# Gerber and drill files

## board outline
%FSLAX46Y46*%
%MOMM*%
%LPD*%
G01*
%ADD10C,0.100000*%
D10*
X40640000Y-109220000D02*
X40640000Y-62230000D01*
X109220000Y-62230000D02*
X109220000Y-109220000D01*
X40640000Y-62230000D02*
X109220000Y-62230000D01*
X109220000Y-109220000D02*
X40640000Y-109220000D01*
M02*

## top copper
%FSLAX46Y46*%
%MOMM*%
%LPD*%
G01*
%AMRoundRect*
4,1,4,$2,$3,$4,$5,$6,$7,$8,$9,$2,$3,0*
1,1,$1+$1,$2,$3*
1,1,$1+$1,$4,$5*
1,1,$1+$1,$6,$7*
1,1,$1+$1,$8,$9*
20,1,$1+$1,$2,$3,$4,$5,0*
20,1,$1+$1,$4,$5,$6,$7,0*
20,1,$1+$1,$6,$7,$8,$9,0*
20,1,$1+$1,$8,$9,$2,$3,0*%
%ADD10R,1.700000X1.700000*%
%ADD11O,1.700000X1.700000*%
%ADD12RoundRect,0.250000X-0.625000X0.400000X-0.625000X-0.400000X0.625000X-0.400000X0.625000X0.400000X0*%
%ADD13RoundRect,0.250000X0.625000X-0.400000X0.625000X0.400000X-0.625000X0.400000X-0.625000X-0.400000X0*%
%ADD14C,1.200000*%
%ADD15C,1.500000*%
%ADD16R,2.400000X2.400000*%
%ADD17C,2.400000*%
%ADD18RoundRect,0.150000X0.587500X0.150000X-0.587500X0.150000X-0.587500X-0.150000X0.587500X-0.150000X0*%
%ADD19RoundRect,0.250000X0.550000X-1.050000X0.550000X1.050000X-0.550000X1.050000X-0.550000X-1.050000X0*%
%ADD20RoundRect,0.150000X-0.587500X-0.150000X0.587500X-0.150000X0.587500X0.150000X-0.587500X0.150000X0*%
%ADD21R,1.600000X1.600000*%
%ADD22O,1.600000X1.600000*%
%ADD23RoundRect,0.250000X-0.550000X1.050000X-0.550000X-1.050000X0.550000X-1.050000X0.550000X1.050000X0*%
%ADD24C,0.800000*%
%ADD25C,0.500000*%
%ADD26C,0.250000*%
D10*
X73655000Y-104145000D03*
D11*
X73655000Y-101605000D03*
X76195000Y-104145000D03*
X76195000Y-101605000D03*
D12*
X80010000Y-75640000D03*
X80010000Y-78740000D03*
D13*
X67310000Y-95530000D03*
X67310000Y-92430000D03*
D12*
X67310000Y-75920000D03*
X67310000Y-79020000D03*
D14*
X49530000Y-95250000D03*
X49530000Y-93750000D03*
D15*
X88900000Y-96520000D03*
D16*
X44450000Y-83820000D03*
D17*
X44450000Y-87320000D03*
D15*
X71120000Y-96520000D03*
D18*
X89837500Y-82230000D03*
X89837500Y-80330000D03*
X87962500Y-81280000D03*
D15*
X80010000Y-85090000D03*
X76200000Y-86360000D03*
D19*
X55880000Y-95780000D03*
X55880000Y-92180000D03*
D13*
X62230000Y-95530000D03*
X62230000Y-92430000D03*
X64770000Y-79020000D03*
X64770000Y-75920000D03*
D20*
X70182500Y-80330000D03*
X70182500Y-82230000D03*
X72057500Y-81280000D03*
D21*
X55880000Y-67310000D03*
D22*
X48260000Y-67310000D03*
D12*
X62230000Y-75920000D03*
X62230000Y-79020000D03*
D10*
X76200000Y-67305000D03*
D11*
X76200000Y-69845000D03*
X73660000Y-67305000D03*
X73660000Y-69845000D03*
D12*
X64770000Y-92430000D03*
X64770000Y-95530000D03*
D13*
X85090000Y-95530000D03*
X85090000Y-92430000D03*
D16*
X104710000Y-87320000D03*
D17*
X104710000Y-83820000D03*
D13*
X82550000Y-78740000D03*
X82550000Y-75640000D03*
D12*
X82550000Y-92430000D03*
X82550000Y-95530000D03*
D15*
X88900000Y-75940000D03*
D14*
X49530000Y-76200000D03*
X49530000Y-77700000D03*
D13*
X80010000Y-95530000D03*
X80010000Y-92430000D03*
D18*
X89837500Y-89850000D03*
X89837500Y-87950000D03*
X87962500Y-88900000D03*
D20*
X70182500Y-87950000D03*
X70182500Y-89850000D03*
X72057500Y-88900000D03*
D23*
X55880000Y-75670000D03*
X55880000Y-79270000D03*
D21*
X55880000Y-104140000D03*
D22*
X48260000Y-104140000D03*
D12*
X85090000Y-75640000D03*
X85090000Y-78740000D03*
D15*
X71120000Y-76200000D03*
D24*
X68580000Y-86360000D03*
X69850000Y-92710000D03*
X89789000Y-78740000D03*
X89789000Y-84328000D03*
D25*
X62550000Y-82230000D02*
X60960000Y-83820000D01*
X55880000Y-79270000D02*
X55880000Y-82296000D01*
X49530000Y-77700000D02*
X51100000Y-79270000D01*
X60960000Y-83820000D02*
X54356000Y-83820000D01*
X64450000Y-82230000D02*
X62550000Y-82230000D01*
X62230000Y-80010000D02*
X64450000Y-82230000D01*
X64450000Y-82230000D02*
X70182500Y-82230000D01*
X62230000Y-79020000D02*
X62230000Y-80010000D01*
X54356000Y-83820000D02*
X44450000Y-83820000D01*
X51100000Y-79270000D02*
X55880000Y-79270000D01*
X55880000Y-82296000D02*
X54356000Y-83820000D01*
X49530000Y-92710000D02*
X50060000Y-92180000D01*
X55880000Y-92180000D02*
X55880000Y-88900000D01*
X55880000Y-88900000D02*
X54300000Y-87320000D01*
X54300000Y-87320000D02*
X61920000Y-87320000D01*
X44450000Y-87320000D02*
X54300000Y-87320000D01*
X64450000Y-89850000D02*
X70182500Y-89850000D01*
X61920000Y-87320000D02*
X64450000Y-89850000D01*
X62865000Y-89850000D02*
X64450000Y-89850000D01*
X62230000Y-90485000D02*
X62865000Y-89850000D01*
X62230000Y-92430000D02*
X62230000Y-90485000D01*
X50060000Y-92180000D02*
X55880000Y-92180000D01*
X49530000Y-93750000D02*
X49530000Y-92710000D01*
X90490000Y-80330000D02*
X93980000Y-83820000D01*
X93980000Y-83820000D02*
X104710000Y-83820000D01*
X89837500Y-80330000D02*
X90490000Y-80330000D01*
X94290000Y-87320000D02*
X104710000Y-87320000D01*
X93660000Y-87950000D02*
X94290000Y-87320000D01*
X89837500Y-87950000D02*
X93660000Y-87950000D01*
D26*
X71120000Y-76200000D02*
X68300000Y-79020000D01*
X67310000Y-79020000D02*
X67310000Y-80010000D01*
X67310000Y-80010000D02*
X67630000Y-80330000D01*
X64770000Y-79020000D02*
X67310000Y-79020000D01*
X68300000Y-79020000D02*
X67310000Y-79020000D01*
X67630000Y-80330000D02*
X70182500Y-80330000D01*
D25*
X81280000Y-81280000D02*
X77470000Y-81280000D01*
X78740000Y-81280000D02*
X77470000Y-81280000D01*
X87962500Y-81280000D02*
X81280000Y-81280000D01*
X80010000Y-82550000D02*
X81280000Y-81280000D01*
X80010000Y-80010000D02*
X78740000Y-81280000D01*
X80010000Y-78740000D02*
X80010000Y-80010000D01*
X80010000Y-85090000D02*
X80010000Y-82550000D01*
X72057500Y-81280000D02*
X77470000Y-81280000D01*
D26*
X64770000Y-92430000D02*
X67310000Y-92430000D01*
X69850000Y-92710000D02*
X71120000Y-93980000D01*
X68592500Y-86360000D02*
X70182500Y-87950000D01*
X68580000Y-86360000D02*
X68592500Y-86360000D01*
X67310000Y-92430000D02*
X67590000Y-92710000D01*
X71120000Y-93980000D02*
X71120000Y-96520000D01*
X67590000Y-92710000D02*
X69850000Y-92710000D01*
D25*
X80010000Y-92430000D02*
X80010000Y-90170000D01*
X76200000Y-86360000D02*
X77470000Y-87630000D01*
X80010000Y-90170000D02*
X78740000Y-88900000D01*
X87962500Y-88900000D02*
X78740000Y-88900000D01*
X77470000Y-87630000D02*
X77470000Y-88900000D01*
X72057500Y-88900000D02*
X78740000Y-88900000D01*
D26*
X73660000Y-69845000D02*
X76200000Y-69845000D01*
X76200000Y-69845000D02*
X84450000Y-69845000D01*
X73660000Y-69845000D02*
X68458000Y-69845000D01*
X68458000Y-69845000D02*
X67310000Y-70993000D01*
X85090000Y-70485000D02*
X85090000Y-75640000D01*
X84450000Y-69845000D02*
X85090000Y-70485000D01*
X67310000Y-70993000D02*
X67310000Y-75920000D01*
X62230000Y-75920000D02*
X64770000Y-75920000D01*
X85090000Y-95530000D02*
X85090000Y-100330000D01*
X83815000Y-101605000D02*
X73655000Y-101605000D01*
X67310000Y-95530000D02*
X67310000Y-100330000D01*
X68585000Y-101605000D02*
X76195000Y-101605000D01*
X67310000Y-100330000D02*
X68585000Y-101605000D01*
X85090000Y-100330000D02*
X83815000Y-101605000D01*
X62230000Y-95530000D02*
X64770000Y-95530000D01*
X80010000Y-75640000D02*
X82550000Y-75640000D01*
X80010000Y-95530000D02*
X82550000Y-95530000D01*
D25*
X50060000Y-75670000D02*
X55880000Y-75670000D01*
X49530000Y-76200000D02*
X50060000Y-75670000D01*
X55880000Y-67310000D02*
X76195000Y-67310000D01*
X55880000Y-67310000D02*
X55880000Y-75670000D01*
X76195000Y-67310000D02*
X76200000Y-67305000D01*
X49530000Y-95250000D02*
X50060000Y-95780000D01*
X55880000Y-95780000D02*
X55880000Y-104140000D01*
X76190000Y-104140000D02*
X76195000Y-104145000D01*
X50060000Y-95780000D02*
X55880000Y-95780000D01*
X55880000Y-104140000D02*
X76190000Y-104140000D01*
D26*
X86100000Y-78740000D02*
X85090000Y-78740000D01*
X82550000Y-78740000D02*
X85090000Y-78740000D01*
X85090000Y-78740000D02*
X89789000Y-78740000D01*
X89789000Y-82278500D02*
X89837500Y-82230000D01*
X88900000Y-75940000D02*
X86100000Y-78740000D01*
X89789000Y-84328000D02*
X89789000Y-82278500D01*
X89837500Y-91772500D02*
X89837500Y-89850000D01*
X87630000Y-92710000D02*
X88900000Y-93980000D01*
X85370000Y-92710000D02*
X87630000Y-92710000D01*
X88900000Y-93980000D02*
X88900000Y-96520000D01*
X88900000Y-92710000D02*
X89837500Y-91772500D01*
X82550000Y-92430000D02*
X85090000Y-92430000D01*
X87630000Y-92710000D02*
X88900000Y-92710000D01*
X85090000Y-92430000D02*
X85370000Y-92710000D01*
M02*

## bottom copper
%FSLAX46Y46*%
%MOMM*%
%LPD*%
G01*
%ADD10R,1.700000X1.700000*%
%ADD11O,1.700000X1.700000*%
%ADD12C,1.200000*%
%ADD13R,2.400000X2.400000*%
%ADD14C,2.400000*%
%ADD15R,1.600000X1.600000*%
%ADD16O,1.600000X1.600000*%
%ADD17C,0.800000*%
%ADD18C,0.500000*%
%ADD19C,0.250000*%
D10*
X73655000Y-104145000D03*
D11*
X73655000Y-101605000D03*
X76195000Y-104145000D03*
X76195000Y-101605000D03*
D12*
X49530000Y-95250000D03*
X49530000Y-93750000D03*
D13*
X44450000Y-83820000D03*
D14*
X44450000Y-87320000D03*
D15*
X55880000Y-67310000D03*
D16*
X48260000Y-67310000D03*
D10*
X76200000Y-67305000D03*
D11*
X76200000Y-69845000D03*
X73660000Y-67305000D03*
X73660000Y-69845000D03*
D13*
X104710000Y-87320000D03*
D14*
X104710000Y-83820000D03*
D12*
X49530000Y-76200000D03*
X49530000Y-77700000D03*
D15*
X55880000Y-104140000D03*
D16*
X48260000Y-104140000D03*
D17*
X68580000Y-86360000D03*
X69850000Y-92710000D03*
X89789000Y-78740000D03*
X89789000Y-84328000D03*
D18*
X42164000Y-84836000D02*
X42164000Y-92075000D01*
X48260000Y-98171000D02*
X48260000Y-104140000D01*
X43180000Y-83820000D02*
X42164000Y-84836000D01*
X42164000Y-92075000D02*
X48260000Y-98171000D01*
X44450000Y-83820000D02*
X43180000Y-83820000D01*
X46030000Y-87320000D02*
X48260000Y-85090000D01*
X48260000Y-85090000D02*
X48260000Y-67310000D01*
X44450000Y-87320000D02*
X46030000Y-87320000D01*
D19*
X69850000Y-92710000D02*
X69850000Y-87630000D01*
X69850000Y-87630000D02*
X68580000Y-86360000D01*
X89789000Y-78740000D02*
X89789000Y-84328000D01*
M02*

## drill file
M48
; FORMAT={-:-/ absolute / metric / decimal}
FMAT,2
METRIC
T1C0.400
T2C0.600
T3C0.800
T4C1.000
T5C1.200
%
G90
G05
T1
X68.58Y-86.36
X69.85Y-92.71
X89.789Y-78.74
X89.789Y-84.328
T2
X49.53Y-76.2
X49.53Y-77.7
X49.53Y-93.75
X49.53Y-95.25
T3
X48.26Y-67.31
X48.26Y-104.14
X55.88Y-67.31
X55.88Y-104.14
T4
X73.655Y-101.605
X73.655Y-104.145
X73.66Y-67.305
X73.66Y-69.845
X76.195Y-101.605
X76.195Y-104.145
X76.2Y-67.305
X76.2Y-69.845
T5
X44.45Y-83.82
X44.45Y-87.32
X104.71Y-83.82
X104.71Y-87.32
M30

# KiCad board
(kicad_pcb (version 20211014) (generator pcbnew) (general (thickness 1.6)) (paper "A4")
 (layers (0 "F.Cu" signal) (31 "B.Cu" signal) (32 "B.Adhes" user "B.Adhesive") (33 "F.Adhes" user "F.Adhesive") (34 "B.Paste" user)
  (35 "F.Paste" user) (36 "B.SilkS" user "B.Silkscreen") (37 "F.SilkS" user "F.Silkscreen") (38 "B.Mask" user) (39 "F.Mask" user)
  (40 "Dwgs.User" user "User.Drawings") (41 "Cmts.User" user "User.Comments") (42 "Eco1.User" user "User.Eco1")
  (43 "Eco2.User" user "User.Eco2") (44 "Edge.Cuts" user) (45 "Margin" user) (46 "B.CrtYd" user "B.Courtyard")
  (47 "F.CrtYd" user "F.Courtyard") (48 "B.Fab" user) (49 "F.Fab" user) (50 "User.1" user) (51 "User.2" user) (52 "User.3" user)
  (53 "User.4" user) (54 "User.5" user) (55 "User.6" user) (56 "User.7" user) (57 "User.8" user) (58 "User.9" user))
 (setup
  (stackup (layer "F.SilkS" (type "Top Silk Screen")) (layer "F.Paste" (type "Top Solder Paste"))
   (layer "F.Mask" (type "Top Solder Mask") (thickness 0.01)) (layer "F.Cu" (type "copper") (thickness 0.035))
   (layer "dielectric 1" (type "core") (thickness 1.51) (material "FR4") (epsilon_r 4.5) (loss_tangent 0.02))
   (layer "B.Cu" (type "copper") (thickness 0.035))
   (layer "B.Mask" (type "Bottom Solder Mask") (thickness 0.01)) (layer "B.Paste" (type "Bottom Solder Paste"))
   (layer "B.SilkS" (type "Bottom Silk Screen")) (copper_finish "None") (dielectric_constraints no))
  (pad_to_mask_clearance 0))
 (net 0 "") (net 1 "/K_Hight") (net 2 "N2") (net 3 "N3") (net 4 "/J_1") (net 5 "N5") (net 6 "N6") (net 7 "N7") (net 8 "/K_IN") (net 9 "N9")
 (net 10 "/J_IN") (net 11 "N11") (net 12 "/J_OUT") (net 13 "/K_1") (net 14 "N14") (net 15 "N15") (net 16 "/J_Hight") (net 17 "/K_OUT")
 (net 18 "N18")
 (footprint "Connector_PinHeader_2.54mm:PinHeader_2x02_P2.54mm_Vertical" (layer "F.Cu") (at 73.655 104.145 90)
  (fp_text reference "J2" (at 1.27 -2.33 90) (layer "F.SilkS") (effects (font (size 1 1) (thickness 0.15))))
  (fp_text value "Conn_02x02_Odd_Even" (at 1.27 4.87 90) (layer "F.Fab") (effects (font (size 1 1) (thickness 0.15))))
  (pad "1" thru_hole rect locked (at 0 0 90) (size 1.7 1.7) (drill 1) (layers *.Cu *.Mask) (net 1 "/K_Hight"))
  (pad "2" thru_hole oval locked (at 2.54 0 90) (size 1.7 1.7) (drill 1) (layers *.Cu *.Mask) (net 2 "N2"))
  (pad "3" thru_hole oval locked (at 0 2.54 90) (size 1.7 1.7) (drill 1) (layers *.Cu *.Mask) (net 1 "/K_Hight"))
  (pad "4" thru_hole oval locked (at 2.54 2.54 90) (size 1.7 1.7) (drill 1) (layers *.Cu *.Mask) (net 2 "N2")))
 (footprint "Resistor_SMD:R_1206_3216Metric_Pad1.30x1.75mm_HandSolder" (layer "F.Cu") (at 80.01 77.19 -90)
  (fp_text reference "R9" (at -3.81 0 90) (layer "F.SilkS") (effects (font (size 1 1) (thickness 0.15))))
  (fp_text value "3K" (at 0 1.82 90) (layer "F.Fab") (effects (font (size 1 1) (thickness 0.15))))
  (pad "1" smd roundrect locked (at -1.55 0 270) (size 1.3 1.75) (layers "F.Cu" "F.Paste" "F.Mask") (roundrect_rratio 0.1923076923)
   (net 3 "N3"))
  (pad "2" smd roundrect locked (at 1.55 0 270) (size 1.3 1.75) (layers "F.Cu" "F.Paste" "F.Mask") (roundrect_rratio 0.1923076923)
   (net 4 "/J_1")))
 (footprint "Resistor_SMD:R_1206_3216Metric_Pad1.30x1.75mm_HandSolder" (layer "F.Cu") (at 67.31 93.98 90)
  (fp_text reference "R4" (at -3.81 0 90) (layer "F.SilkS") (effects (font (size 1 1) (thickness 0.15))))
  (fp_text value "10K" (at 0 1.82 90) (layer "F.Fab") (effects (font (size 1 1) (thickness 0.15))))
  (pad "1" smd roundrect locked (at -1.55 0 90) (size 1.3 1.75) (layers "F.Cu" "F.Paste" "F.Mask") (roundrect_rratio 0.1923076923)
   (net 2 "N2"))
  (pad "2" smd roundrect locked (at 1.55 0 90) (size 1.3 1.75) (layers "F.Cu" "F.Paste" "F.Mask") (roundrect_rratio 0.1923076923)
   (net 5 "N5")))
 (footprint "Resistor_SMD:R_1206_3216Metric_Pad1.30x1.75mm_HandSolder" (layer "F.Cu") (at 67.31 77.47 -90)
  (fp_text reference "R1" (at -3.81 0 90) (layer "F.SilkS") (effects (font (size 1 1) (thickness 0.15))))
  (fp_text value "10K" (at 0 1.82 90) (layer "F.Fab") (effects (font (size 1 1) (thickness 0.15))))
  (pad "1" smd roundrect locked (at -1.55 0 270) (size 1.3 1.75) (layers "F.Cu" "F.Paste" "F.Mask") (roundrect_rratio 0.1923076923)
   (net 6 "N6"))
  (pad "2" smd roundrect locked (at 1.55 0 270) (size 1.3 1.75) (layers "F.Cu" "F.Paste" "F.Mask") (roundrect_rratio 0.1923076923)
   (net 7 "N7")))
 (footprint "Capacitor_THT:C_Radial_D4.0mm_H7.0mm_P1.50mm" (layer "F.Cu") (at 49.53 95.25 90)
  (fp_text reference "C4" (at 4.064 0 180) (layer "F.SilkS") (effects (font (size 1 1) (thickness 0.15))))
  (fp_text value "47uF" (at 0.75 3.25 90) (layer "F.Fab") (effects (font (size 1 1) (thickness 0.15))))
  (pad "1" thru_hole circle locked (at 0 0 90) (size 1.2 1.2) (drill 0.6) (layers *.Cu *.Mask) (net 1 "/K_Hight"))
  (pad "2" thru_hole circle locked (at 1.5 0 90) (size 1.2 1.2) (drill 0.6) (layers *.Cu *.Mask) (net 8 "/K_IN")))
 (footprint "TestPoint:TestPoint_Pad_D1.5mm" (layer "F.Cu") (at 88.9 96.52)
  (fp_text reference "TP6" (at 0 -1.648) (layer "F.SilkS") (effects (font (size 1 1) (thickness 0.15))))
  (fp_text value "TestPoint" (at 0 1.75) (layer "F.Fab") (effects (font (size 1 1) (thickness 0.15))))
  (pad "1" smd circle locked (at 0 0) (size 1.5 1.5) (layers "F.Cu" "F.Mask") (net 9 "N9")))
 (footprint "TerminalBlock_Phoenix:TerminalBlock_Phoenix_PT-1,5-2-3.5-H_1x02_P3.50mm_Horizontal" (layer "F.Cu") (at 44.45 83.82 -90)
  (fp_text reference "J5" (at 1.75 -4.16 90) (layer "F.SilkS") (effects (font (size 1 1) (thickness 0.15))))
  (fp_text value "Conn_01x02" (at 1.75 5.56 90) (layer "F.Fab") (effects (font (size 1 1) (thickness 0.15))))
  (pad "1" thru_hole rect locked (at 0 0 270) (size 2.4 2.4) (drill 1.2) (layers *.Cu *.Mask) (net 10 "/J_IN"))
  (pad "2" thru_hole circle locked (at 3.5 0 270) (size 2.4 2.4) (drill 1.2) (layers *.Cu *.Mask) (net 8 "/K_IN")))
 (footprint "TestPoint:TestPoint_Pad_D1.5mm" (layer "F.Cu") (at 71.12 96.52)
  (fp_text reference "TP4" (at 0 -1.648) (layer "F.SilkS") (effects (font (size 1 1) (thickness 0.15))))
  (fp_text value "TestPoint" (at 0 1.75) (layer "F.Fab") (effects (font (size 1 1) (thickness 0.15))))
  (pad "1" smd circle locked (at 0 0) (size 1.5 1.5) (layers "F.Cu" "F.Mask") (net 5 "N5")))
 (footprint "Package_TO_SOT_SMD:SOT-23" (layer "F.Cu") (at 88.9 81.28 180)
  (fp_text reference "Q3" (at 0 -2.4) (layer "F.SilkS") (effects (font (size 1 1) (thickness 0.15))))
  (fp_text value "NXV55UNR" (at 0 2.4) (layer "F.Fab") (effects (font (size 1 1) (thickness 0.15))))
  (pad "1" smd roundrect locked (at -0.9375 -0.95 180) (size 1.475 0.6) (layers "F.Cu" "F.Paste" "F.Mask") (roundrect_rratio 0.25)
   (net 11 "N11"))
  (pad "2" smd roundrect locked (at -0.9375 0.95 180) (size 1.475 0.6) (layers "F.Cu" "F.Paste" "F.Mask") (roundrect_rratio 0.25)
   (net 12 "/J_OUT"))
  (pad "3" smd roundrect locked (at 0.9375 0 180) (size 1.475 0.6) (layers "F.Cu" "F.Paste" "F.Mask") (roundrect_rratio 0.25) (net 4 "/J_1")))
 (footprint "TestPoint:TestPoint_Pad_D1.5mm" (layer "F.Cu") (at 80.01 85.09)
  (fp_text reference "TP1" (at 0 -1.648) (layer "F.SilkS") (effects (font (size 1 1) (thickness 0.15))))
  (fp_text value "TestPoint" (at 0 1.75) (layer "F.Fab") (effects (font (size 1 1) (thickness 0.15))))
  (pad "1" smd circle locked (at 0 0) (size 1.5 1.5) (layers "F.Cu" "F.Mask") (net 4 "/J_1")))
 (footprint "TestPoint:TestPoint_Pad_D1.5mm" (layer "F.Cu") (at 76.2 86.36)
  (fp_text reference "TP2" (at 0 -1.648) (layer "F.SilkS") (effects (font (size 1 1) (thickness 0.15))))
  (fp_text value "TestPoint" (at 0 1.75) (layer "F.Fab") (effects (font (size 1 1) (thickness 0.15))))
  (pad "1" smd circle locked (at 0 0) (size 1.5 1.5) (layers "F.Cu" "F.Mask") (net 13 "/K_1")))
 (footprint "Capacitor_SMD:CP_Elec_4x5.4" (layer "F.Cu") (at 55.88 93.98 90)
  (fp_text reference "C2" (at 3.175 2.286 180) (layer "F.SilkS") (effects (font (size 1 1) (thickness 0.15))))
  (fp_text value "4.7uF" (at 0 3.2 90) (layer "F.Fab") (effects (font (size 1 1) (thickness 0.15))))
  (pad "1" smd roundrect locked (at -1.8 0 90) (size 2.6 1.6) (layers "F.Cu" "F.Paste" "F.Mask") (roundrect_rratio 0.15625)
   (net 1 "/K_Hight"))
  (pad "2" smd roundrect locked (at 1.8 0 90) (size 2.6 1.6) (layers "F.Cu" "F.Paste" "F.Mask") (roundrect_rratio 0.15625) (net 8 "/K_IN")))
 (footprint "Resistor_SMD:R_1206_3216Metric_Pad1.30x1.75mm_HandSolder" (layer "F.Cu") (at 62.23 93.98 90)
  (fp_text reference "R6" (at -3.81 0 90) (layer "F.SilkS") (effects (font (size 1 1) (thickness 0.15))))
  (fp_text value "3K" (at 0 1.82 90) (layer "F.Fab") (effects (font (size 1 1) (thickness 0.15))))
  (pad "1" smd roundrect locked (at -1.55 0 90) (size 1.3 1.75) (layers "F.Cu" "F.Paste" "F.Mask") (roundrect_rratio 0.1923076923)
   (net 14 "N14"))
  (pad "2" smd roundrect locked (at 1.55 0 90) (size 1.3 1.75) (layers "F.Cu" "F.Paste" "F.Mask") (roundrect_rratio 0.1923076923)
   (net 8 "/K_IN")))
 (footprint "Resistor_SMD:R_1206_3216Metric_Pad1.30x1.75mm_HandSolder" (layer "F.Cu") (at 64.77 77.47 90)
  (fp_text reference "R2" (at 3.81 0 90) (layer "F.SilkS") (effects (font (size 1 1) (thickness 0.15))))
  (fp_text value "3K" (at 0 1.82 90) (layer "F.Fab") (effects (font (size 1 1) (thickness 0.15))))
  (pad "1" smd roundrect locked (at -1.55 0 90) (size 1.3 1.75) (layers "F.Cu" "F.Paste" "F.Mask") (roundrect_rratio 0.1923076923)
   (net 7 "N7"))
  (pad "2" smd roundrect locked (at 1.55 0 90) (size 1.3 1.75) (layers "F.Cu" "F.Paste" "F.Mask") (roundrect_rratio 0.1923076923)
   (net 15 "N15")))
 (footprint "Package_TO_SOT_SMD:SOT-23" (layer "F.Cu") (at 71.12 81.28)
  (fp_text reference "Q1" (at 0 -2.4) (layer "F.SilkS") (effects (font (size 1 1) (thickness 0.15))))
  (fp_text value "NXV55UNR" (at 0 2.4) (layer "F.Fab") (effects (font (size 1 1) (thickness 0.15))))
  (pad "1" smd roundrect locked (at -0.9375 -0.95) (size 1.475 0.6) (layers "F.Cu" "F.Paste" "F.Mask") (roundrect_rratio 0.25) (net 7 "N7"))
  (pad "2" smd roundrect locked (at -0.9375 0.95) (size 1.475 0.6) (layers "F.Cu" "F.Paste" "F.Mask") (roundrect_rratio 0.25)
   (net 10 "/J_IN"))
  (pad "3" smd roundrect locked (at 0.9375 0) (size 1.475 0.6) (layers "F.Cu" "F.Paste" "F.Mask") (roundrect_rratio 0.25) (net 4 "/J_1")))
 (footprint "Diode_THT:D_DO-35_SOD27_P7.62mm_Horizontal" (layer "F.Cu") (at 55.88 67.31 180)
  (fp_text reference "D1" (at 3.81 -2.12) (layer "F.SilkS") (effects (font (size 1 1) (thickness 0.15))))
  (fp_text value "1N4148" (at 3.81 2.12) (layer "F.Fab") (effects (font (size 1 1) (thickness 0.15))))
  (pad "1" thru_hole rect locked (at 0 0 180) (size 1.6 1.6) (drill 0.8) (layers *.Cu *.Mask) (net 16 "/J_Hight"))
  (pad "2" thru_hole oval locked (at 7.62 0 180) (size 1.6 1.6) (drill 0.8) (layers *.Cu *.Mask) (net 8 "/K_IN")))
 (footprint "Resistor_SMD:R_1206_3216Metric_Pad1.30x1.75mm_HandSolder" (layer "F.Cu") (at 62.23 77.47 -90)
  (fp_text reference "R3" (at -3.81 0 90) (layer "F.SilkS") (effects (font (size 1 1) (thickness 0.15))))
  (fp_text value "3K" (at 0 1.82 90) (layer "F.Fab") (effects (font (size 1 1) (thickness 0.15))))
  (pad "1" smd roundrect locked (at -1.55 0 270) (size 1.3 1.75) (layers "F.Cu" "F.Paste" "F.Mask") (roundrect_rratio 0.1923076923)
   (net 15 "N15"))
  (pad "2" smd roundrect locked (at 1.55 0 270) (size 1.3 1.75) (layers "F.Cu" "F.Paste" "F.Mask") (roundrect_rratio 0.1923076923)
   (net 10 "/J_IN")))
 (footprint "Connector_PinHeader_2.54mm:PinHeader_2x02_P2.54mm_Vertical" (layer "F.Cu") (at 76.2 67.305 -90) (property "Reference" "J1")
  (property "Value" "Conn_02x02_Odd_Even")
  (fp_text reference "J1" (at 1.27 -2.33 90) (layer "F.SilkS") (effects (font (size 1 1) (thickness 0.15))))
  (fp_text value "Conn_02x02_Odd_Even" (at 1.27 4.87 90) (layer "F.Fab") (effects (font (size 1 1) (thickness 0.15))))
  (pad "1" thru_hole rect locked (at 0 0 270) (size 1.7 1.7) (drill 1) (layers *.Cu *.Mask) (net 16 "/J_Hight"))
  (pad "2" thru_hole oval locked (at 2.54 0 270) (size 1.7 1.7) (drill 1) (layers *.Cu *.Mask) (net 6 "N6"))
  (pad "3" thru_hole oval locked (at 0 2.54 270) (size 1.7 1.7) (drill 1) (layers *.Cu *.Mask) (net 16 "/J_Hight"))
  (pad "4" thru_hole oval locked (at 2.54 2.54 270) (size 1.7 1.7) (drill 1) (layers *.Cu *.Mask) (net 6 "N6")))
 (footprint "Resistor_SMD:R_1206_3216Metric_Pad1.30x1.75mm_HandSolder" (layer "F.Cu") (at 64.77 93.98 -90)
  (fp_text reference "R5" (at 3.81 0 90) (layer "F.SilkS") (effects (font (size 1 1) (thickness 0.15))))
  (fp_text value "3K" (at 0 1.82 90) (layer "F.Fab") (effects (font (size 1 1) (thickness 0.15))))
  (pad "1" smd roundrect locked (at -1.55 0 270) (size 1.3 1.75) (layers "F.Cu" "F.Paste" "F.Mask") (roundrect_rratio 0.1923076923)
   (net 5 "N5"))
  (pad "2" smd roundrect locked (at 1.55 0 270) (size 1.3 1.75) (layers "F.Cu" "F.Paste" "F.Mask") (roundrect_rratio 0.1923076923)
   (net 14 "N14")))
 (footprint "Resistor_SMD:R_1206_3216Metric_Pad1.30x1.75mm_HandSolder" (layer "F.Cu") (at 85.09 93.98 90)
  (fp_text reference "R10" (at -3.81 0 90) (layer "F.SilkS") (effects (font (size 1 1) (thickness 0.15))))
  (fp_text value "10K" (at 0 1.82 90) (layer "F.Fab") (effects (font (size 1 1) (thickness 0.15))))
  (pad "1" smd roundrect locked (at -1.55 0 90) (size 1.3 1.75) (layers "F.Cu" "F.Paste" "F.Mask") (roundrect_rratio 0.1923076923)
   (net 2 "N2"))
  (pad "2" smd roundrect locked (at 1.55 0 90) (size 1.3 1.75) (layers "F.Cu" "F.Paste" "F.Mask") (roundrect_rratio 0.1923076923)
   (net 9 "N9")))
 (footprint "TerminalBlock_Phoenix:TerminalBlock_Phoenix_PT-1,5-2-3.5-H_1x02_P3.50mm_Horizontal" (layer "F.Cu") (at 104.71 87.32 90)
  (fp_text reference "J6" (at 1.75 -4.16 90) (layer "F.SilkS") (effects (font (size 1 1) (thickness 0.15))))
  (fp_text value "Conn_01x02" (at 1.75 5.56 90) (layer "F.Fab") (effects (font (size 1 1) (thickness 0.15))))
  (pad "1" thru_hole rect locked (at 0 0 90) (size 2.4 2.4) (drill 1.2) (layers *.Cu *.Mask) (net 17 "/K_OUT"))
  (pad "2" thru_hole circle locked (at 3.5 0 90) (size 2.4 2.4) (drill 1.2) (layers *.Cu *.Mask) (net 12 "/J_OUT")))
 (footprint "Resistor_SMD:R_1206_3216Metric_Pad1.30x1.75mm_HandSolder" (layer "F.Cu") (at 82.55 77.19 90)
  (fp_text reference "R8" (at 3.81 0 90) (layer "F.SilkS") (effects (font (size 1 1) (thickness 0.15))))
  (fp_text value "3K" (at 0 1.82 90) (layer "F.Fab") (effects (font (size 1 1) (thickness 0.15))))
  (pad "1" smd roundrect locked (at -1.55 0 90) (size 1.3 1.75) (layers "F.Cu" "F.Paste" "F.Mask") (roundrect_rratio 0.1923076923)
   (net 11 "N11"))
  (pad "2" smd roundrect locked (at 1.55 0 90) (size 1.3 1.75) (layers "F.Cu" "F.Paste" "F.Mask") (roundrect_rratio 0.1923076923)
   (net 3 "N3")))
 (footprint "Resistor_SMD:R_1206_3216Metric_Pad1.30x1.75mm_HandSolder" (layer "F.Cu") (at 82.55 93.98 -90)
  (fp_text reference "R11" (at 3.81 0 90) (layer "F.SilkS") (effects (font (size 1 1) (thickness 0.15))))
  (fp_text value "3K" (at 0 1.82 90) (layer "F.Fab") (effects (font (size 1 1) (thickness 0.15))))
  (pad "1" smd roundrect locked (at -1.55 0 270) (size 1.3 1.75) (layers "F.Cu" "F.Paste" "F.Mask") (roundrect_rratio 0.1923076923)
   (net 9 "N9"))
  (pad "2" smd roundrect locked (at 1.55 0 270) (size 1.3 1.75) (layers "F.Cu" "F.Paste" "F.Mask") (roundrect_rratio 0.1923076923)
   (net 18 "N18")))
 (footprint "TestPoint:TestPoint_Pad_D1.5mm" (layer "F.Cu") (at 88.9 75.94)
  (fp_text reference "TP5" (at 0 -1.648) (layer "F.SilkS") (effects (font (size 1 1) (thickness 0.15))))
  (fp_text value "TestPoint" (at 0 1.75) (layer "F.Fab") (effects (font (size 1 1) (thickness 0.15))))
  (pad "1" smd circle locked (at 0 0) (size 1.5 1.5) (layers "F.Cu" "F.Mask") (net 11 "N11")))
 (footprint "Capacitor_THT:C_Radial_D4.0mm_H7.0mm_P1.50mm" (layer "F.Cu") (at 49.53 76.2 -90)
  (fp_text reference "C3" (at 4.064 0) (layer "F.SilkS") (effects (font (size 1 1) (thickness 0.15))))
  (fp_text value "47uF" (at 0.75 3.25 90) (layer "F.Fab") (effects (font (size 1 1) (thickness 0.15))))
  (pad "1" thru_hole circle locked (at 0 0 270) (size 1.2 1.2) (drill 0.6) (layers *.Cu *.Mask) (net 16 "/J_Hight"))
  (pad "2" thru_hole circle locked (at 1.5 0 270) (size 1.2 1.2) (drill 0.6) (layers *.Cu *.Mask) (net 10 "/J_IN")))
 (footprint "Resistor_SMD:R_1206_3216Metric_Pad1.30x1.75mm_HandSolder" (layer "F.Cu") (at 80.01 93.98 90)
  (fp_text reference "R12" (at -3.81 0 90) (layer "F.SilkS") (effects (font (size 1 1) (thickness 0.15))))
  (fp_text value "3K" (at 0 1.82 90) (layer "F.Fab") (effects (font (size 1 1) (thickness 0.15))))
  (pad "1" smd roundrect locked (at -1.55 0 90) (size 1.3 1.75) (layers "F.Cu" "F.Paste" "F.Mask") (roundrect_rratio 0.1923076923)
   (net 18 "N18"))
  (pad "2" smd roundrect locked (at 1.55 0 90) (size 1.3 1.75) (layers "F.Cu" "F.Paste" "F.Mask") (roundrect_rratio 0.1923076923)
   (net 13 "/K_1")))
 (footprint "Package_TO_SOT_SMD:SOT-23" (layer "F.Cu") (at 88.9 88.9 180)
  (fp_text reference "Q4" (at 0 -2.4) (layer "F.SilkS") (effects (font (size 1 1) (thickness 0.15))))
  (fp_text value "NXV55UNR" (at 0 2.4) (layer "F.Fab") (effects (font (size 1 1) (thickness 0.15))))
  (pad "1" smd roundrect locked (at -0.9375 -0.95 180) (size 1.475 0.6) (layers "F.Cu" "F.Paste" "F.Mask") (roundrect_rratio 0.25)
   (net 9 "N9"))
  (pad "2" smd roundrect locked (at -0.9375 0.95 180) (size 1.475 0.6) (layers "F.Cu" "F.Paste" "F.Mask") (roundrect_rratio 0.25)
   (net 17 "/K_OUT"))
  (pad "3" smd roundrect locked (at 0.9375 0 180) (size 1.475 0.6) (layers "F.Cu" "F.Paste" "F.Mask") (roundrect_rratio 0.25)
   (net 13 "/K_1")))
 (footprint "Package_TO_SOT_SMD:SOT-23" (layer "F.Cu") (at 71.12 88.9)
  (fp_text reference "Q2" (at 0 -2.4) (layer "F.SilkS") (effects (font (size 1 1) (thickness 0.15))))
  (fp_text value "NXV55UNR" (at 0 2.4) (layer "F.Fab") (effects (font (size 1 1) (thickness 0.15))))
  (pad "1" smd roundrect locked (at -0.9375 -0.95) (size 1.475 0.6) (layers "F.Cu" "F.Paste" "F.Mask") (roundrect_rratio 0.25) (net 5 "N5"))
  (pad "2" smd roundrect locked (at -0.9375 0.95) (size 1.475 0.6) (layers "F.Cu" "F.Paste" "F.Mask") (roundrect_rratio 0.25)
   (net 8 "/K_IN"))
  (pad "3" smd roundrect locked (at 0.9375 0) (size 1.475 0.6) (layers "F.Cu" "F.Paste" "F.Mask") (roundrect_rratio 0.25) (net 13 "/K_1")))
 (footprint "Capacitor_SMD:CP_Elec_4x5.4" (layer "F.Cu") (at 55.88 77.47 -90)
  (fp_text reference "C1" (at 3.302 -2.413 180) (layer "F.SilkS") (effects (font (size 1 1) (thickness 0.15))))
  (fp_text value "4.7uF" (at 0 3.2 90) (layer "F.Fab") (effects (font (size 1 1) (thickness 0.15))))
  (pad "1" smd roundrect locked (at -1.8 0 270) (size 2.6 1.6) (layers "F.Cu" "F.Paste" "F.Mask") (roundrect_rratio 0.15625)
   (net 16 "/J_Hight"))
  (pad "2" smd roundrect locked (at 1.8 0 270) (size 2.6 1.6) (layers "F.Cu" "F.Paste" "F.Mask") (roundrect_rratio 0.15625) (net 10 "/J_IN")))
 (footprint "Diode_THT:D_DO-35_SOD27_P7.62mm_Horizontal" (layer "F.Cu") (at 55.88 104.14 180)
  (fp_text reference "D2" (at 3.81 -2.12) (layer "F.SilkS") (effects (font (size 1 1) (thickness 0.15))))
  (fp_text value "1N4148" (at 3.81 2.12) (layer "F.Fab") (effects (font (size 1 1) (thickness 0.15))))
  (pad "1" thru_hole rect locked (at 0 0 180) (size 1.6 1.6) (drill 0.8) (layers *.Cu *.Mask) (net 1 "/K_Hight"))
  (pad "2" thru_hole oval locked (at 7.62 0 180) (size 1.6 1.6) (drill 0.8) (layers *.Cu *.Mask) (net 10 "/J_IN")))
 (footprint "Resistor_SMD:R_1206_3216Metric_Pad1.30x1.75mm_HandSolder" (layer "F.Cu") (at 85.09 77.19 -90)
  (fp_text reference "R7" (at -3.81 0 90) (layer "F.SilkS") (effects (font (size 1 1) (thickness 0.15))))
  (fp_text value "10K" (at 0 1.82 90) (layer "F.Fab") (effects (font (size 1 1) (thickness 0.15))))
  (pad "1" smd roundrect locked (at -1.55 0 270) (size 1.3 1.75) (layers "F.Cu" "F.Paste" "F.Mask") (roundrect_rratio 0.1923076923)
   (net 6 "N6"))
  (pad "2" smd roundrect locked (at 1.55 0 270) (size 1.3 1.75) (layers "F.Cu" "F.Paste" "F.Mask") (roundrect_rratio 0.1923076923)
   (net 11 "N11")))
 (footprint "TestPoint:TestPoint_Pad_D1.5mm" (layer "F.Cu") (at 71.12 76.2)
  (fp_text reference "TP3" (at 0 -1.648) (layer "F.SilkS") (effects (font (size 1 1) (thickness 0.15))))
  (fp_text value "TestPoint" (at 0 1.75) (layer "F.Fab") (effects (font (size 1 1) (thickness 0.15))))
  (pad "1" smd circle locked (at 0 0) (size 1.5 1.5) (layers "F.Cu" "F.Mask") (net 7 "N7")))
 (gr_line (start 40.64 109.22) (end 40.64 62.23) (layer "Edge.Cuts") (width 0.1))
 (gr_line (start 109.22 62.23) (end 109.22 109.22) (layer "Edge.Cuts") (width 0.1))
 (gr_line (start 40.64 62.23) (end 109.22 62.23) (layer "Edge.Cuts") (width 0.1))
 (gr_line (start 109.22 109.22) (end 40.64 109.22) (layer "Edge.Cuts") (width 0.1))
 (segment (start 62.55 82.23) (end 60.96 83.82) (width 0.5) (layer "F.Cu") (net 10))
 (segment (start 55.88 79.27) (end 55.88 82.296) (width 0.5) (layer "F.Cu") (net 10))
 (segment (start 49.53 77.7) (end 51.1 79.27) (width 0.5) (layer "F.Cu") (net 10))
 (segment (start 60.96 83.82) (end 54.356 83.82) (width 0.5) (layer "F.Cu") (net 10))
 (segment (start 64.45 82.23) (end 62.55 82.23) (width 0.5) (layer "F.Cu") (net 10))
 (segment (start 62.23 80.01) (end 64.45 82.23) (width 0.5) (layer "F.Cu") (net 10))
 (segment (start 64.45 82.23) (end 70.1825 82.23) (width 0.5) (layer "F.Cu") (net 10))
 (segment (start 62.23 79.02) (end 62.23 80.01) (width 0.5) (layer "F.Cu") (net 10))
 (segment (start 54.356 83.82) (end 44.45 83.82) (width 0.5) (layer "F.Cu") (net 10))
 (segment (start 51.1 79.27) (end 55.88 79.27) (width 0.5) (layer "F.Cu") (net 10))
 (segment (start 55.88 82.296) (end 54.356 83.82) (width 0.5) (layer "F.Cu") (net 10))
 (segment (start 42.164 84.836) (end 42.164 92.075) (width 0.5) (layer "B.Cu") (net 10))
 (segment (start 48.26 98.171) (end 48.26 104.14) (width 0.5) (layer "B.Cu") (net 10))
 (segment (start 43.18 83.82) (end 42.164 84.836) (width 0.5) (layer "B.Cu") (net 10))
 (segment (start 42.164 92.075) (end 48.26 98.171) (width 0.5) (layer "B.Cu") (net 10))
 (segment (start 44.45 83.82) (end 43.18 83.82) (width 0.5) (layer "B.Cu") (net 10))
 (segment (start 49.53 92.71) (end 50.06 92.18) (width 0.5) (layer "F.Cu") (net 8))
 (segment (start 55.88 92.18) (end 55.88 88.9) (width 0.5) (layer "F.Cu") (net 8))
 (segment (start 55.88 88.9) (end 54.3 87.32) (width 0.5) (layer "F.Cu") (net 8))
 (segment (start 54.3 87.32) (end 61.92 87.32) (width 0.5) (layer "F.Cu") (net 8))
 (segment (start 44.45 87.32) (end 54.3 87.32) (width 0.5) (layer "F.Cu") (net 8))
 (segment (start 64.45 89.85) (end 70.1825 89.85) (width 0.5) (layer "F.Cu") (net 8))
 (segment (start 61.92 87.32) (end 64.45 89.85) (width 0.5) (layer "F.Cu") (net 8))
 (segment (start 62.865 89.85) (end 64.45 89.85) (width 0.5) (layer "F.Cu") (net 8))
 (segment (start 62.23 90.485) (end 62.865 89.85) (width 0.5) (layer "F.Cu") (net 8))
 (segment (start 62.23 92.43) (end 62.23 90.485) (width 0.5) (layer "F.Cu") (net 8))
 (segment (start 50.06 92.18) (end 55.88 92.18) (width 0.5) (layer "F.Cu") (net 8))
 (segment (start 49.53 93.75) (end 49.53 92.71) (width 0.5) (layer "F.Cu") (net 8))
 (segment (start 46.03 87.32) (end 48.26 85.09) (width 0.5) (layer "B.Cu") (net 8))
 (segment (start 48.26 85.09) (end 48.26 67.31) (width 0.5) (layer "B.Cu") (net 8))
 (segment (start 44.45 87.32) (end 46.03 87.32) (width 0.5) (layer "B.Cu") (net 8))
 (segment (start 90.49 80.33) (end 93.98 83.82) (width 0.5) (layer "F.Cu") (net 12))
 (segment (start 93.98 83.82) (end 104.71 83.82) (width 0.5) (layer "F.Cu") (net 12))
 (segment (start 89.8375 80.33) (end 90.49 80.33) (width 0.5) (layer "F.Cu") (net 12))
 (segment (start 94.29 87.32) (end 104.71 87.32) (width 0.5) (layer "F.Cu") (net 17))
 (segment (start 93.66 87.95) (end 94.29 87.32) (width 0.5) (layer "F.Cu") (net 17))
 (segment (start 89.8375 87.95) (end 93.66 87.95) (width 0.5) (layer "F.Cu") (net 17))
 (segment (start 71.12 76.2) (end 68.3 79.02) (width 0.25) (layer "F.Cu") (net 7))
 (segment (start 67.31 79.02) (end 67.31 80.01) (width 0.25) (layer "F.Cu") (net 7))
 (segment (start 67.31 80.01) (end 67.63 80.33) (width 0.25) (layer "F.Cu") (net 7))
 (segment (start 64.77 79.02) (end 67.31 79.02) (width 0.25) (layer "F.Cu") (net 7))
 (segment (start 68.3 79.02) (end 67.31 79.02) (width 0.25) (layer "F.Cu") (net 7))
 (segment (start 67.63 80.33) (end 70.1825 80.33) (width 0.25) (layer "F.Cu") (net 7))
 (segment (start 81.28 81.28) (end 77.47 81.28) (width 0.5) (layer "F.Cu") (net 4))
 (segment (start 78.74 81.28) (end 77.47 81.28) (width 0.5) (layer "F.Cu") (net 4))
 (segment (start 87.9625 81.28) (end 81.28 81.28) (width 0.5) (layer "F.Cu") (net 4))
 (segment (start 80.01 82.55) (end 81.28 81.28) (width 0.5) (layer "F.Cu") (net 4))
 (segment (start 80.01 80.01) (end 78.74 81.28) (width 0.5) (layer "F.Cu") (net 4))
 (segment (start 80.01 78.74) (end 80.01 80.01) (width 0.5) (layer "F.Cu") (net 4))
 (segment (start 80.01 85.09) (end 80.01 82.55) (width 0.5) (layer "F.Cu") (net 4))
 (segment (start 72.0575 81.28) (end 77.47 81.28) (width 0.5) (layer "F.Cu") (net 4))
 (segment (start 64.77 92.43) (end 67.31 92.43) (width 0.25) (layer "F.Cu") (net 5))
 (segment (start 69.85 92.71) (end 71.12 93.98) (width 0.25) (layer "F.Cu") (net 5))
 (segment (start 68.5925 86.36) (end 70.1825 87.95) (width 0.25) (layer "F.Cu") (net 5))
 (segment (start 68.58 86.36) (end 68.5925 86.36) (width 0.25) (layer "F.Cu") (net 5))
 (segment (start 67.31 92.43) (end 67.59 92.71) (width 0.25) (layer "F.Cu") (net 5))
 (segment (start 71.12 93.98) (end 71.12 96.52) (width 0.25) (layer "F.Cu") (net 5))
 (segment (start 67.59 92.71) (end 69.85 92.71) (width 0.25) (layer "F.Cu") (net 5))
 (via (at 68.58 86.36) (size 0.8) (drill 0.4) (layers "F.Cu" "B.Cu") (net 5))
 (via (at 69.85 92.71) (size 0.8) (drill 0.4) (layers "F.Cu" "B.Cu") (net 5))
 (segment (start 69.85 92.71) (end 69.85 87.63) (width 0.25) (layer "B.Cu") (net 5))
 (segment (start 69.85 87.63) (end 68.58 86.36) (width 0.25) (layer "B.Cu") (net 5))
 (segment (start 80.01 92.43) (end 80.01 90.17) (width 0.5) (layer "F.Cu") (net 13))
 (segment (start 76.2 86.36) (end 77.47 87.63) (width 0.5) (layer "F.Cu") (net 13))
 (segment (start 80.01 90.17) (end 78.74 88.9) (width 0.5) (layer "F.Cu") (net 13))
 (segment (start 87.9625 88.9) (end 78.74 88.9) (width 0.5) (layer "F.Cu") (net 13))
 (segment (start 77.47 87.63) (end 77.47 88.9) (width 0.5) (layer "F.Cu") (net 13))
 (segment (start 72.0575 88.9) (end 78.74 88.9) (width 0.5) (layer "F.Cu") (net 13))
 (segment (start 73.66 69.845) (end 76.2 69.845) (width 0.25) (layer "F.Cu") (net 6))
 (segment (start 76.2 69.845) (end 84.45 69.845) (width 0.25) (layer "F.Cu") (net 6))
 (segment (start 73.66 69.845) (end 68.458 69.845) (width 0.25) (layer "F.Cu") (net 6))
 (segment (start 68.458 69.845) (end 67.31 70.993) (width 0.25) (layer "F.Cu") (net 6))
 (segment (start 85.09 70.485) (end 85.09 75.64) (width 0.25) (layer "F.Cu") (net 6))
 (segment (start 84.45 69.845) (end 85.09 70.485) (width 0.25) (layer "F.Cu") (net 6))
 (segment (start 67.31 70.993) (end 67.31 75.92) (width 0.25) (layer "F.Cu") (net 6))
 (segment (start 62.23 75.92) (end 64.77 75.92) (width 0.25) (layer "F.Cu") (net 15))
 (segment (start 85.09 95.53) (end 85.09 100.33) (width 0.25) (layer "F.Cu") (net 2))
 (segment (start 83.815 101.605) (end 73.655 101.605) (width 0.25) (layer "F.Cu") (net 2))
 (segment (start 67.31 95.53) (end 67.31 100.33) (width 0.25) (layer "F.Cu") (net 2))
 (segment (start 68.585 101.605) (end 76.195 101.605) (width 0.25) (layer "F.Cu") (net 2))
 (segment (start 67.31 100.33) (end 68.585 101.605) (width 0.25) (layer "F.Cu") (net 2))
 (segment (start 85.09 100.33) (end 83.815 101.605) (width 0.25) (layer "F.Cu") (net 2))
 (segment (start 62.23 95.53) (end 64.77 95.53) (width 0.25) (layer "F.Cu") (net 14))
 (segment (start 80.01 75.64) (end 82.55 75.64) (width 0.25) (layer "F.Cu") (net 3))
 (segment (start 80.01 95.53) (end 82.55 95.53) (width 0.25) (layer "F.Cu") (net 18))
 (segment (start 50.06 75.67) (end 55.88 75.67) (width 0.5) (layer "F.Cu") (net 16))
 (segment (start 49.53 76.2) (end 50.06 75.67) (width 0.5) (layer "F.Cu") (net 16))
 (segment (start 55.88 67.31) (end 76.195 67.31) (width 0.5) (layer "F.Cu") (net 16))
 (segment (start 55.88 67.31) (end 55.88 75.67) (width 0.5) (layer "F.Cu") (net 16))
 (segment (start 76.195 67.31) (end 76.2 67.305) (width 0.5) (layer "F.Cu") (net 16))
 (segment (start 49.53 95.25) (end 50.06 95.78) (width 0.5) (layer "F.Cu") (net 1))
 (segment (start 55.88 95.78) (end 55.88 104.14) (width 0.5) (layer "F.Cu") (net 1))
 (segment (start 76.19 104.14) (end 76.195 104.145) (width 0.5) (layer "F.Cu") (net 1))
 (segment (start 50.06 95.78) (end 55.88 95.78) (width 0.5) (layer "F.Cu") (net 1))
 (segment (start 55.88 104.14) (end 76.19 104.14) (width 0.5) (layer "F.Cu") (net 1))
 (segment (start 86.1 78.74) (end 85.09 78.74) (width 0.25) (layer "F.Cu") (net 11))
 (segment (start 82.55 78.74) (end 85.09 78.74) (width 0.25) (layer "F.Cu") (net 11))
 (segment (start 85.09 78.74) (end 89.789 78.74) (width 0.25) (layer "F.Cu") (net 11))
 (segment (start 89.789 82.2785) (end 89.8375 82.23) (width 0.25) (layer "F.Cu") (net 11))
 (segment (start 88.9 75.94) (end 86.1 78.74) (width 0.25) (layer "F.Cu") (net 11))
 (segment (start 89.789 84.328) (end 89.789 82.2785) (width 0.25) (layer "F.Cu") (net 11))
 (via (at 89.789 78.74) (size 0.8) (drill 0.4) (layers "F.Cu" "B.Cu") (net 11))
 (via (at 89.789 84.328) (size 0.8) (drill 0.4) (layers "F.Cu" "B.Cu") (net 11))
 (segment (start 89.789 78.74) (end 89.789 84.328) (width 0.25) (layer "B.Cu") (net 11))
 (segment (start 89.8375 91.7725) (end 89.8375 89.85) (width 0.25) (layer "F.Cu") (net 9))
 (segment (start 87.63 92.71) (end 88.9 93.98) (width 0.25) (layer "F.Cu") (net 9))
 (segment (start 85.37 92.71) (end 87.63 92.71) (width 0.25) (layer "F.Cu") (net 9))
 (segment (start 88.9 93.98) (end 88.9 96.52) (width 0.25) (layer "F.Cu") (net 9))
 (segment (start 88.9 92.71) (end 89.8375 91.7725) (width 0.25) (layer "F.Cu") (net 9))
 (segment (start 82.55 92.43) (end 85.09 92.43) (width 0.25) (layer "F.Cu") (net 9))
 (segment (start 87.63 92.71) (end 88.9 92.71) (width 0.25) (layer "F.Cu") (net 9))
 (segment (start 85.09 92.43) (end 85.37 92.71) (width 0.25) (layer "F.Cu") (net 9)))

